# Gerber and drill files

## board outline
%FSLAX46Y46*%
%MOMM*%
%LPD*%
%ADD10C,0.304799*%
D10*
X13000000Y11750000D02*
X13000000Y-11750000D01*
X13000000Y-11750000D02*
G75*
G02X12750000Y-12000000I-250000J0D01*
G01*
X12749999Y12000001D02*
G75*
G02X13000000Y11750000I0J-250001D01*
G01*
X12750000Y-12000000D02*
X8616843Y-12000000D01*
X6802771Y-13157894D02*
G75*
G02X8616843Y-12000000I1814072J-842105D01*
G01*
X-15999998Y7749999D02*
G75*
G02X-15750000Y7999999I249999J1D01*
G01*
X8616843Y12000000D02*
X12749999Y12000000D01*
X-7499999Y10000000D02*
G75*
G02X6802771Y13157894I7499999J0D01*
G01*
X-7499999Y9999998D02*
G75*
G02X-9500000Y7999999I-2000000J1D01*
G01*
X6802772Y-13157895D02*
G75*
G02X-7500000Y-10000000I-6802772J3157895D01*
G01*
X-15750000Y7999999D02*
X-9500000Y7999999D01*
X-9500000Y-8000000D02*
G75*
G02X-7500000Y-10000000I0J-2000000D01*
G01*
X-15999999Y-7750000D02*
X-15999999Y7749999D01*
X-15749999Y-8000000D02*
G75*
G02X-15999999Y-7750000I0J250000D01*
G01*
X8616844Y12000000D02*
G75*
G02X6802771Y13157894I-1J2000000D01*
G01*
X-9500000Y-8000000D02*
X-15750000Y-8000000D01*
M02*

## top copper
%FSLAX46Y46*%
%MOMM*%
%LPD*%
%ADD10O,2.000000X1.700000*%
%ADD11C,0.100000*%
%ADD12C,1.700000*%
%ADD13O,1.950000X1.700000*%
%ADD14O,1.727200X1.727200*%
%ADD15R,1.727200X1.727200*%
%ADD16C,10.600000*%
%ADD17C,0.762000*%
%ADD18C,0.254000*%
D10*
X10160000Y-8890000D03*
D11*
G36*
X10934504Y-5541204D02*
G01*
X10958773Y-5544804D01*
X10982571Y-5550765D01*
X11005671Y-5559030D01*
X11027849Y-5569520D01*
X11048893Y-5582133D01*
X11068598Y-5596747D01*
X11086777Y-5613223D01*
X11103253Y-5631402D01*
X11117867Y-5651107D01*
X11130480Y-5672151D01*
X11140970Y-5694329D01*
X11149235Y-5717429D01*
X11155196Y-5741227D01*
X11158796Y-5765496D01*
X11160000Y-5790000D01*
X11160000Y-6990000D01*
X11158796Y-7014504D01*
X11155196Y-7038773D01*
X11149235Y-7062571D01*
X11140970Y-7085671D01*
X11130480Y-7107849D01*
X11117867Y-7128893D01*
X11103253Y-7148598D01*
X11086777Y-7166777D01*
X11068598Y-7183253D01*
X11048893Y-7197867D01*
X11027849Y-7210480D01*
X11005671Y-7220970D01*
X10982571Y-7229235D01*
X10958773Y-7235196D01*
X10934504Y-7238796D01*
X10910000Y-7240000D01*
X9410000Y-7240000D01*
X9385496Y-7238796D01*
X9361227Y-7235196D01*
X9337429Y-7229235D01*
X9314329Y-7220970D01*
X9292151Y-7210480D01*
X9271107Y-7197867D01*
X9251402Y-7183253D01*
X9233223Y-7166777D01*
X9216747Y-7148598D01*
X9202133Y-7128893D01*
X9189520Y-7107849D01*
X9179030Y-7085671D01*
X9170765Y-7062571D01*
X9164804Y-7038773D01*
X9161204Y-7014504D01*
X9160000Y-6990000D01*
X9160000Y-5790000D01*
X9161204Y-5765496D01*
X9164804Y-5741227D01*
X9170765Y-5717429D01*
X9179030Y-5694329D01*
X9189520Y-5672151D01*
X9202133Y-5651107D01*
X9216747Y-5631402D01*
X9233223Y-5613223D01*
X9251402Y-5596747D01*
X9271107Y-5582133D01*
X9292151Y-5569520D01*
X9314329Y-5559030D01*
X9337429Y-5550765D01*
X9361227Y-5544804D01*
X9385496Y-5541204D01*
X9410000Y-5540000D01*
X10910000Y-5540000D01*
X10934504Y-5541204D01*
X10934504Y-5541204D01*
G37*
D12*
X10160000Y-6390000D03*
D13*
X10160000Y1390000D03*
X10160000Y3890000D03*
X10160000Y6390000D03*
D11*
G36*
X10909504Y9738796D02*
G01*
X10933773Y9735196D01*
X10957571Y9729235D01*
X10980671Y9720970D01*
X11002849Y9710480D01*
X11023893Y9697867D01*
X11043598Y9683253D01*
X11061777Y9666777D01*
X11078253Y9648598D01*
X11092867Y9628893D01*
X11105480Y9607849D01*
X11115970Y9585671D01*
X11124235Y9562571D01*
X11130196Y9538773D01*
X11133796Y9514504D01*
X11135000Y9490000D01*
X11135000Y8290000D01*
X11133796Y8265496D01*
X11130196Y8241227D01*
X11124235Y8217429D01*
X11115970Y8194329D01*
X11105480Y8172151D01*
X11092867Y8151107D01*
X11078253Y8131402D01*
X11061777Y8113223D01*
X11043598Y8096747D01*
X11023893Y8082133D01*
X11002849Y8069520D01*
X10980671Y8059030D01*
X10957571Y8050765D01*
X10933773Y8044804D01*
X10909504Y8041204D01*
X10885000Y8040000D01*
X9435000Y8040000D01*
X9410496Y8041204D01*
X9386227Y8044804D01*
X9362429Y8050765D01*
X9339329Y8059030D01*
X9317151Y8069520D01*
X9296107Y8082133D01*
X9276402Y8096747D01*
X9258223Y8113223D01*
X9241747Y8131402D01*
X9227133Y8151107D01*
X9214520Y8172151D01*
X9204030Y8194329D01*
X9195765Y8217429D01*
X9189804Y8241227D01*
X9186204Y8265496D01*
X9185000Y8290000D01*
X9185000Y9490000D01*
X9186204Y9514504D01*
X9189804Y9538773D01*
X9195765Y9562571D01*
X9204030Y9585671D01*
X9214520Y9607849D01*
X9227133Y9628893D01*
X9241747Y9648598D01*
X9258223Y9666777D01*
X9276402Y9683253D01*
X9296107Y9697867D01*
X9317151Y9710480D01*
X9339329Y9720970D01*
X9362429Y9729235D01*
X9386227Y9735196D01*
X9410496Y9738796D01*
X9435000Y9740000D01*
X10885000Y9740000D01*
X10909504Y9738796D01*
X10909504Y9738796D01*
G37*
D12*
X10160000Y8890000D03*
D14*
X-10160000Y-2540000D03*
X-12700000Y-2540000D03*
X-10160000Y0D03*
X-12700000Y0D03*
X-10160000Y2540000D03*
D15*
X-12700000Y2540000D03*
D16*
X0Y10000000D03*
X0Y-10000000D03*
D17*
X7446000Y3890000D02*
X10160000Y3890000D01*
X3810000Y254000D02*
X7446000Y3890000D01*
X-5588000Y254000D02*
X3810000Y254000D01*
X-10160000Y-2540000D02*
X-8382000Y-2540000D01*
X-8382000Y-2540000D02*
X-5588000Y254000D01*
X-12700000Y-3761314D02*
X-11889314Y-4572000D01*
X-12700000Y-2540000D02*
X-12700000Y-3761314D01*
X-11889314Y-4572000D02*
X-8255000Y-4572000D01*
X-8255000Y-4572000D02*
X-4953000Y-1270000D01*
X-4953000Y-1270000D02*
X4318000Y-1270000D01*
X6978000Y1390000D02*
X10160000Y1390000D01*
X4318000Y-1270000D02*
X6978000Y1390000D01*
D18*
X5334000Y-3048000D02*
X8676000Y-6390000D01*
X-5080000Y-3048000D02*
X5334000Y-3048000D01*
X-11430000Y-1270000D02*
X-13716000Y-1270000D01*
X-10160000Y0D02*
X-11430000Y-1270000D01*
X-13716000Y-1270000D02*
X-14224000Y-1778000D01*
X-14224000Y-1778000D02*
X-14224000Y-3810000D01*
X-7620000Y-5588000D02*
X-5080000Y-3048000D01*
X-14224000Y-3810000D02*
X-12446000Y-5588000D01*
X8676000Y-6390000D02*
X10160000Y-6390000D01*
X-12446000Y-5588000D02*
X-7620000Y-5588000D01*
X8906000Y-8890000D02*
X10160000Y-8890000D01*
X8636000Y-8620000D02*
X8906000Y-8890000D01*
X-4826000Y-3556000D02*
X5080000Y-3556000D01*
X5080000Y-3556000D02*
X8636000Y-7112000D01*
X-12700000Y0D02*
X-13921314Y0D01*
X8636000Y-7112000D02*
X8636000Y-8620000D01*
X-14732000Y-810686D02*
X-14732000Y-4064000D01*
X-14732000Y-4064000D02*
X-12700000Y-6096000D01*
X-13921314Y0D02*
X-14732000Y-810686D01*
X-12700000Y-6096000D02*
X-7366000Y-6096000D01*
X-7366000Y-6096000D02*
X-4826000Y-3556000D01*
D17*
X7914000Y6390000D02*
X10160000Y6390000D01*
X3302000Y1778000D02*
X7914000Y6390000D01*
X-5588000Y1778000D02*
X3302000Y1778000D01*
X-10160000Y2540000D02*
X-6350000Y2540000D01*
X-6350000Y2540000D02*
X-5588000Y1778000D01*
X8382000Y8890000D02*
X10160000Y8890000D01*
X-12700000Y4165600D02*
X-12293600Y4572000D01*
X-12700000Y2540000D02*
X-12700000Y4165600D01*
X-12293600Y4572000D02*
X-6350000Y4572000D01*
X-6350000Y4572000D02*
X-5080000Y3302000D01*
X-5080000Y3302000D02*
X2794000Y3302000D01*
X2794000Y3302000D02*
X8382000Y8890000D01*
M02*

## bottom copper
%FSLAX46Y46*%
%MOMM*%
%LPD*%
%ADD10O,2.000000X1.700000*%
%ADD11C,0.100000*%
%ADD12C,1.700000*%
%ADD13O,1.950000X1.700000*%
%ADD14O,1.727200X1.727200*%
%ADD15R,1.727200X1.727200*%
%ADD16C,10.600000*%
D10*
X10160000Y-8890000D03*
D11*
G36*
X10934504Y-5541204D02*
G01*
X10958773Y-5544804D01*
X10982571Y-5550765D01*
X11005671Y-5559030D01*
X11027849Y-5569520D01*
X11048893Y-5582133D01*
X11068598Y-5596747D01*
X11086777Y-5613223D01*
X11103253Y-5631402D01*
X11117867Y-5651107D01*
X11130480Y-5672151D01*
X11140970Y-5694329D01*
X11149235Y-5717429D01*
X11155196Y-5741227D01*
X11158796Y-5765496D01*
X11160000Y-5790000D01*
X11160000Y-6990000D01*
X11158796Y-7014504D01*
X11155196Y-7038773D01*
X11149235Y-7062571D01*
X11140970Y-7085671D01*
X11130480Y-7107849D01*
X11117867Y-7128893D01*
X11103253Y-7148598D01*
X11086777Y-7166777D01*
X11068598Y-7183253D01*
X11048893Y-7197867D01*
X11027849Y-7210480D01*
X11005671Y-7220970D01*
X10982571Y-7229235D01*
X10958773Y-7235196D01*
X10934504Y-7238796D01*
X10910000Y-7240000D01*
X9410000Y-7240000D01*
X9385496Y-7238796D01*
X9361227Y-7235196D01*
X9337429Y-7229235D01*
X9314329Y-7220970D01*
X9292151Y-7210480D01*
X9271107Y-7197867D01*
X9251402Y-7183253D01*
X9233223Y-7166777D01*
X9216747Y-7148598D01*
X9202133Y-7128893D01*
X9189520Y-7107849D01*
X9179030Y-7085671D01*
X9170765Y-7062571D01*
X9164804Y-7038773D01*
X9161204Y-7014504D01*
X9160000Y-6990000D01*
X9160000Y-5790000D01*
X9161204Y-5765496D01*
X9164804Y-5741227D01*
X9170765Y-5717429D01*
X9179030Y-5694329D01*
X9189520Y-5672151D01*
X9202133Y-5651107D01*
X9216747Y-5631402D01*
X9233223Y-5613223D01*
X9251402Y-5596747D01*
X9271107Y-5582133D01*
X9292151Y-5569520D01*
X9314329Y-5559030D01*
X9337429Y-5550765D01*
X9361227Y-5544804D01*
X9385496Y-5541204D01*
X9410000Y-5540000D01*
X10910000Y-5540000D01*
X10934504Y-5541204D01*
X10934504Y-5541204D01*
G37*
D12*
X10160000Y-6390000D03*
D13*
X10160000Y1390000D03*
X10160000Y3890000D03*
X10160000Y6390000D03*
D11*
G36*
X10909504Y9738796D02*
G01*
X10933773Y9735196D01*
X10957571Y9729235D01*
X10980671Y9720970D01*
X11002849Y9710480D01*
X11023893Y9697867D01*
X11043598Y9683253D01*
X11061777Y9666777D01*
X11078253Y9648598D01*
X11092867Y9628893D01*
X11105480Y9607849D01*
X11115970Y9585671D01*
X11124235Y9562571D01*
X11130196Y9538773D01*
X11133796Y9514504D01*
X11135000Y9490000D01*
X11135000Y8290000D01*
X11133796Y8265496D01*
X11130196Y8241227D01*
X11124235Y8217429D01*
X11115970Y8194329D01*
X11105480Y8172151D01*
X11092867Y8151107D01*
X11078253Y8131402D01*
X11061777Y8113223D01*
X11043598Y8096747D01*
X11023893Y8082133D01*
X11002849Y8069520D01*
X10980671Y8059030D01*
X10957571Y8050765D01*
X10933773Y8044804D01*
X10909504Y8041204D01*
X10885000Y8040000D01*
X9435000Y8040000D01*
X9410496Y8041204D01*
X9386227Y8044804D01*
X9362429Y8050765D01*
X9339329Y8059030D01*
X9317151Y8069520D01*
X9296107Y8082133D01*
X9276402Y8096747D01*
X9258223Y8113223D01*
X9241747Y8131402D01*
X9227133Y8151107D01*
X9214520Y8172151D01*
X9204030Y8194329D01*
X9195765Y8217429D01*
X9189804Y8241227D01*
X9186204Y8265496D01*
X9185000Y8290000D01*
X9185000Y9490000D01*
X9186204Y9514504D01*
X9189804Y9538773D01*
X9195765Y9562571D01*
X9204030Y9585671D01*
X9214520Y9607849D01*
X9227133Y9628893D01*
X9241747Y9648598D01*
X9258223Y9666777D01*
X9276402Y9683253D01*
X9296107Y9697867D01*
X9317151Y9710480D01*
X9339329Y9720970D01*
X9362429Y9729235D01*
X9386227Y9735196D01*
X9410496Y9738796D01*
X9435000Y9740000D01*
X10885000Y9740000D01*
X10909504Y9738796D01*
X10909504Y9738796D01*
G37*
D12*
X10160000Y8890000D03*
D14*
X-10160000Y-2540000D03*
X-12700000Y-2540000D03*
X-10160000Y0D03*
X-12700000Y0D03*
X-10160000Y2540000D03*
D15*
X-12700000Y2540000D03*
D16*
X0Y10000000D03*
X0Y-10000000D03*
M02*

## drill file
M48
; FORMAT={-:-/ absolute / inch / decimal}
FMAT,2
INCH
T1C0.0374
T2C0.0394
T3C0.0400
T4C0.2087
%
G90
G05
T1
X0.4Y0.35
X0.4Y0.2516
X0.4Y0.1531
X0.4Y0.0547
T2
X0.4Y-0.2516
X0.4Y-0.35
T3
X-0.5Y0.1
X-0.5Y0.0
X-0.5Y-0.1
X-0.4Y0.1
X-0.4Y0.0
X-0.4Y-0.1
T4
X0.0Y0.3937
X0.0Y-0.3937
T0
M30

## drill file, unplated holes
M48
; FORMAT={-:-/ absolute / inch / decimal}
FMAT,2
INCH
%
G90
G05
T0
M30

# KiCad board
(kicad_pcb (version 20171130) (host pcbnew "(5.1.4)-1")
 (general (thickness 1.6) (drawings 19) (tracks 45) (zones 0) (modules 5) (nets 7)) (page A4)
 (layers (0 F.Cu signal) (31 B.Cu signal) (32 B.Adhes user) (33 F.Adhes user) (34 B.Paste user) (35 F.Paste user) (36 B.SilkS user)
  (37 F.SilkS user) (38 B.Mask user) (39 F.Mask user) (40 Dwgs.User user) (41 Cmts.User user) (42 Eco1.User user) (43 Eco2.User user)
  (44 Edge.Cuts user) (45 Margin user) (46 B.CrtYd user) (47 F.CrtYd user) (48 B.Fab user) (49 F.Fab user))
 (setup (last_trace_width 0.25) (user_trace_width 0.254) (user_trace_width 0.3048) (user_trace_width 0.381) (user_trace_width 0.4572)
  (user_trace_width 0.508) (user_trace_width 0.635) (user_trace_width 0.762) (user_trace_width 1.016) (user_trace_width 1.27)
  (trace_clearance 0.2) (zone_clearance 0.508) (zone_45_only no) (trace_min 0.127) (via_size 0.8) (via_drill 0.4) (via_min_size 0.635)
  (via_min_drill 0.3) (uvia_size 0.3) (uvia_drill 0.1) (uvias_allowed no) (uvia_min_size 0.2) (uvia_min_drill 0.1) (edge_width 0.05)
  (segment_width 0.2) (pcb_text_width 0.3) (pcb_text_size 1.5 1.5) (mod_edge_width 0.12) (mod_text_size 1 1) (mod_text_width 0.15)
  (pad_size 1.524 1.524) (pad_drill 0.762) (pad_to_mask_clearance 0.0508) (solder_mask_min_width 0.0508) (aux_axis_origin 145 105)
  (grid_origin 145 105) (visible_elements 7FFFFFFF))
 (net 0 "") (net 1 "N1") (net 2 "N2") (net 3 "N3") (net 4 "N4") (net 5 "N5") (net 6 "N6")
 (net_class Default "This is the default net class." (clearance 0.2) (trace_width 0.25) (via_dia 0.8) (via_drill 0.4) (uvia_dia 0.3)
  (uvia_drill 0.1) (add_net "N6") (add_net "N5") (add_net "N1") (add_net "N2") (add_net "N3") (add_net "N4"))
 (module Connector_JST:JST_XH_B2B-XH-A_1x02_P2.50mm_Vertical (layer F.Cu) (at 155.16 111.39 270)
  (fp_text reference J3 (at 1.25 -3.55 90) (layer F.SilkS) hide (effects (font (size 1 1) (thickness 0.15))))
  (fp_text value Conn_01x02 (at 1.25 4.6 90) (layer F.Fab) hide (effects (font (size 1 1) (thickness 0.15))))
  (pad 2 thru_hole oval (at 2.5 0 270) (size 1.7 2) (drill 1) (layers *.Cu *.Mask) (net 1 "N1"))
  (pad 1 thru_hole roundrect (at 0 0 270) (size 1.7 2) (drill 1) (layers *.Cu *.Mask) (roundrect_rratio 0.147059) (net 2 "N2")))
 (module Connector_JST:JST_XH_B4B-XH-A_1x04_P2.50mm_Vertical (layer F.Cu) (at 155.16 96.11 270)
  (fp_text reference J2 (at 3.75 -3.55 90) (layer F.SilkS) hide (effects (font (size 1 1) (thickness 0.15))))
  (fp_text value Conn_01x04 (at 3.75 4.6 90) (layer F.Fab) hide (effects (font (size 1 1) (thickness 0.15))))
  (pad 4 thru_hole oval (at 7.5 0 270) (size 1.7 1.95) (drill 0.95) (layers *.Cu *.Mask) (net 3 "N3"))
  (pad 3 thru_hole oval (at 5 0 270) (size 1.7 1.95) (drill 0.95) (layers *.Cu *.Mask) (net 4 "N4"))
  (pad 2 thru_hole oval (at 2.5 0 270) (size 1.7 1.95) (drill 0.95) (layers *.Cu *.Mask) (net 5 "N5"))
  (pad 1 thru_hole roundrect (at 0 0 270) (size 1.7 1.95) (drill 0.95) (layers *.Cu *.Mask) (roundrect_rratio 0.147059) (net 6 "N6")))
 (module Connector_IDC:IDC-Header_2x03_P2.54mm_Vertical (layer F.Cu) (at 132.3 102.46)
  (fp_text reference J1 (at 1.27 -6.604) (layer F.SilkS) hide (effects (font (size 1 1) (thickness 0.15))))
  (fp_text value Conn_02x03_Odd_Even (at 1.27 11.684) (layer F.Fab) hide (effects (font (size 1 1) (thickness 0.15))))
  (pad 6 thru_hole oval (at 2.54 5.08) (size 1.7272 1.7272) (drill 1.016) (layers *.Cu *.Mask) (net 4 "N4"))
  (pad 5 thru_hole oval (at 0 5.08) (size 1.7272 1.7272) (drill 1.016) (layers *.Cu *.Mask) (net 3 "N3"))
  (pad 4 thru_hole oval (at 2.54 2.54) (size 1.7272 1.7272) (drill 1.016) (layers *.Cu *.Mask) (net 2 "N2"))
  (pad 3 thru_hole oval (at 0 2.54) (size 1.7272 1.7272) (drill 1.016) (layers *.Cu *.Mask) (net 1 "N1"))
  (pad 2 thru_hole oval (at 2.54 0) (size 1.7272 1.7272) (drill 1.016) (layers *.Cu *.Mask) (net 5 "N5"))
  (pad 1 thru_hole rect (at 0 0) (size 1.7272 1.7272) (drill 1.016) (layers *.Cu *.Mask) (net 6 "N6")))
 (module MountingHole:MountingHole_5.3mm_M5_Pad (layer F.Cu) (at 145 95)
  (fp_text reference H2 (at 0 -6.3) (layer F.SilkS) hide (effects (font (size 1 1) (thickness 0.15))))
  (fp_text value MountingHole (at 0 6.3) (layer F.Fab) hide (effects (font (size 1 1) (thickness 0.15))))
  (pad 1 thru_hole circle (at 0 0) (size 10.6 10.6) (drill 5.3) (layers *.Cu *.Mask)))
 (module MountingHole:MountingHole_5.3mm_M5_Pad (layer F.Cu) (at 145 115)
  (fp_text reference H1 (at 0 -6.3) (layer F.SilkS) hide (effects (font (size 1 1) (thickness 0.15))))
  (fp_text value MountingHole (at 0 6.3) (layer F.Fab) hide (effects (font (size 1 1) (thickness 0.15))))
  (pad 1 thru_hole circle (at 0 0) (size 10.6 10.6) (drill 5.3) (layers *.Cu *.Mask)))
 (gr_line (start 158 93.25) (end 158 116.75) (layer Edge.Cuts) (width 0.304799))
 (gr_arc (start 157.75 116.75) (end 157.75 117) (angle -90) (layer Edge.Cuts) (width 0.304799))
 (gr_arc (start 157.749999 93.25) (end 158 93.25) (angle -90) (layer Edge.Cuts) (width 0.304799))
 (gr_line (start 157.75 117) (end 153.616843 117) (layer Edge.Cuts) (width 0.304799))
 (gr_arc (start 153.616843 118.999999) (end 153.616843 117) (angle -65.09893763) (layer Edge.Cuts) (width 0.304799))
 (gr_arc (start 129.250001 97.25) (end 129.25 97.000001) (angle -90) (layer Edge.Cuts) (width 0.304799))
 (gr_line (start 153.616843 93) (end 157.749999 93) (layer Edge.Cuts) (width 0.304799))
 (gr_arc (start 145 95) (end 151.802771 91.842106) (angle -155.0989376) (layer Edge.Cuts) (width 0.304799))
 (gr_arc (start 135.500001 95.000001) (end 135.5 97.000001) (angle -90) (layer Edge.Cuts) (width 0.304799))
 (gr_arc (start 145 115) (end 137.5 115) (angle -155.0989376) (layer Edge.Cuts) (width 0.304799))
 (gr_line (start 129.25 97.000001) (end 135.5 97.000001) (layer Edge.Cuts) (width 0.304799))
 (gr_arc (start 135.5 115) (end 137.5 115) (angle -90) (layer Edge.Cuts) (width 0.304799))
 (gr_line (start 129.000001 112.75) (end 129.000001 97.250001) (layer Edge.Cuts) (width 0.304799))
 (gr_arc (start 129.250001 112.75) (end 129.000001 112.75) (angle -90) (layer Edge.Cuts) (width 0.304799))
 (gr_arc (start 153.616843 91) (end 151.802771 91.842106) (angle -65.09893763) (layer Edge.Cuts) (width 0.304799))
 (gr_line (start 135.5 113) (end 129.25 113) (layer Edge.Cuts) (width 0.304799))
 (segment (start 152.446 101.11) (end 155.16 101.11) (width 0.762) (layer F.Cu) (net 4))
 (segment (start 148.81 104.746) (end 152.446 101.11) (width 0.762) (layer F.Cu) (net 4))
 (segment (start 139.412 104.746) (end 148.81 104.746) (width 0.762) (layer F.Cu) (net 4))
 (segment (start 134.84 107.54) (end 136.618 107.54) (width 0.762) (layer F.Cu) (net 4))
 (segment (start 136.618 107.54) (end 139.412 104.746) (width 0.762) (layer F.Cu) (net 4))
 (segment (start 132.3 108.761314) (end 133.110686 109.572) (width 0.762) (layer F.Cu) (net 3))
 (segment (start 132.3 107.54) (end 132.3 108.761314) (width 0.762) (layer F.Cu) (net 3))
 (segment (start 133.110686 109.572) (end 136.745 109.572) (width 0.762) (layer F.Cu) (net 3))
 (segment (start 136.745 109.572) (end 140.047 106.27) (width 0.762) (layer F.Cu) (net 3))
 (segment (start 140.047 106.27) (end 149.318 106.27) (width 0.762) (layer F.Cu) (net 3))
 (segment (start 151.978 103.61) (end 155.16 103.61) (width 0.762) (layer F.Cu) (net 3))
 (segment (start 149.318 106.27) (end 151.978 103.61) (width 0.762) (layer F.Cu) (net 3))
 (segment (start 150.334 108.048) (end 153.676 111.39) (width 0.254) (layer F.Cu) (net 2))
 (segment (start 139.92 108.048) (end 150.334 108.048) (width 0.254) (layer F.Cu) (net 2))
 (segment (start 133.57 106.27) (end 131.284 106.27) (width 0.254) (layer F.Cu) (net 2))
 (segment (start 134.84 105) (end 133.57 106.27) (width 0.254) (layer F.Cu) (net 2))
 (segment (start 131.284 106.27) (end 130.776 106.778) (width 0.254) (layer F.Cu) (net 2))
 (segment (start 130.776 106.778) (end 130.776 108.81) (width 0.254) (layer F.Cu) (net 2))
 (segment (start 137.38 110.588) (end 139.92 108.048) (width 0.254) (layer F.Cu) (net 2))
 (segment (start 130.776 108.81) (end 132.554 110.588) (width 0.254) (layer F.Cu) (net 2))
 (segment (start 153.676 111.39) (end 155.16 111.39) (width 0.254) (layer F.Cu) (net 2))
 (segment (start 132.554 110.588) (end 137.38 110.588) (width 0.254) (layer F.Cu) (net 2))
 (segment (start 153.906 113.89) (end 155.16 113.89) (width 0.254) (layer F.Cu) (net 1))
 (segment (start 153.636 113.62) (end 153.906 113.89) (width 0.254) (layer F.Cu) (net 1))
 (segment (start 140.174 108.556) (end 150.08 108.556) (width 0.254) (layer F.Cu) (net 1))
 (segment (start 150.08 108.556) (end 153.636 112.112) (width 0.254) (layer F.Cu) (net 1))
 (segment (start 132.3 105) (end 131.078686 105) (width 0.254) (layer F.Cu) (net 1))
 (segment (start 153.636 112.112) (end 153.636 113.62) (width 0.254) (layer F.Cu) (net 1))
 (segment (start 130.268 105.810686) (end 130.268 109.064) (width 0.254) (layer F.Cu) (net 1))
 (segment (start 130.268 109.064) (end 132.3 111.096) (width 0.254) (layer F.Cu) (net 1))
 (segment (start 131.078686 105) (end 130.268 105.810686) (width 0.254) (layer F.Cu) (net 1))
 (segment (start 132.3 111.096) (end 137.634 111.096) (width 0.254) (layer F.Cu) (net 1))
 (segment (start 137.634 111.096) (end 140.174 108.556) (width 0.254) (layer F.Cu) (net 1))
 (segment (start 152.914 98.61) (end 155.16 98.61) (width 0.762) (layer F.Cu) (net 5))
 (segment (start 148.302 103.222) (end 152.914 98.61) (width 0.762) (layer F.Cu) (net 5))
 (segment (start 139.412 103.222) (end 148.302 103.222) (width 0.762) (layer F.Cu) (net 5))
 (segment (start 134.84 102.46) (end 138.65 102.46) (width 0.762) (layer F.Cu) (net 5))
 (segment (start 138.65 102.46) (end 139.412 103.222) (width 0.762) (layer F.Cu) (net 5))
 (segment (start 153.382 96.11) (end 155.16 96.11) (width 0.762) (layer F.Cu) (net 6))
 (segment (start 132.3 100.8344) (end 132.7064 100.428) (width 0.762) (layer F.Cu) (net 6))
 (segment (start 132.3 102.46) (end 132.3 100.8344) (width 0.762) (layer F.Cu) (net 6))
 (segment (start 132.7064 100.428) (end 138.65 100.428) (width 0.762) (layer F.Cu) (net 6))
 (segment (start 138.65 100.428) (end 139.92 101.698) (width 0.762) (layer F.Cu) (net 6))
 (segment (start 139.92 101.698) (end 147.794 101.698) (width 0.762) (layer F.Cu) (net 6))
 (segment (start 147.794 101.698) (end 153.382 96.11) (width 0.762) (layer F.Cu) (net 6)))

